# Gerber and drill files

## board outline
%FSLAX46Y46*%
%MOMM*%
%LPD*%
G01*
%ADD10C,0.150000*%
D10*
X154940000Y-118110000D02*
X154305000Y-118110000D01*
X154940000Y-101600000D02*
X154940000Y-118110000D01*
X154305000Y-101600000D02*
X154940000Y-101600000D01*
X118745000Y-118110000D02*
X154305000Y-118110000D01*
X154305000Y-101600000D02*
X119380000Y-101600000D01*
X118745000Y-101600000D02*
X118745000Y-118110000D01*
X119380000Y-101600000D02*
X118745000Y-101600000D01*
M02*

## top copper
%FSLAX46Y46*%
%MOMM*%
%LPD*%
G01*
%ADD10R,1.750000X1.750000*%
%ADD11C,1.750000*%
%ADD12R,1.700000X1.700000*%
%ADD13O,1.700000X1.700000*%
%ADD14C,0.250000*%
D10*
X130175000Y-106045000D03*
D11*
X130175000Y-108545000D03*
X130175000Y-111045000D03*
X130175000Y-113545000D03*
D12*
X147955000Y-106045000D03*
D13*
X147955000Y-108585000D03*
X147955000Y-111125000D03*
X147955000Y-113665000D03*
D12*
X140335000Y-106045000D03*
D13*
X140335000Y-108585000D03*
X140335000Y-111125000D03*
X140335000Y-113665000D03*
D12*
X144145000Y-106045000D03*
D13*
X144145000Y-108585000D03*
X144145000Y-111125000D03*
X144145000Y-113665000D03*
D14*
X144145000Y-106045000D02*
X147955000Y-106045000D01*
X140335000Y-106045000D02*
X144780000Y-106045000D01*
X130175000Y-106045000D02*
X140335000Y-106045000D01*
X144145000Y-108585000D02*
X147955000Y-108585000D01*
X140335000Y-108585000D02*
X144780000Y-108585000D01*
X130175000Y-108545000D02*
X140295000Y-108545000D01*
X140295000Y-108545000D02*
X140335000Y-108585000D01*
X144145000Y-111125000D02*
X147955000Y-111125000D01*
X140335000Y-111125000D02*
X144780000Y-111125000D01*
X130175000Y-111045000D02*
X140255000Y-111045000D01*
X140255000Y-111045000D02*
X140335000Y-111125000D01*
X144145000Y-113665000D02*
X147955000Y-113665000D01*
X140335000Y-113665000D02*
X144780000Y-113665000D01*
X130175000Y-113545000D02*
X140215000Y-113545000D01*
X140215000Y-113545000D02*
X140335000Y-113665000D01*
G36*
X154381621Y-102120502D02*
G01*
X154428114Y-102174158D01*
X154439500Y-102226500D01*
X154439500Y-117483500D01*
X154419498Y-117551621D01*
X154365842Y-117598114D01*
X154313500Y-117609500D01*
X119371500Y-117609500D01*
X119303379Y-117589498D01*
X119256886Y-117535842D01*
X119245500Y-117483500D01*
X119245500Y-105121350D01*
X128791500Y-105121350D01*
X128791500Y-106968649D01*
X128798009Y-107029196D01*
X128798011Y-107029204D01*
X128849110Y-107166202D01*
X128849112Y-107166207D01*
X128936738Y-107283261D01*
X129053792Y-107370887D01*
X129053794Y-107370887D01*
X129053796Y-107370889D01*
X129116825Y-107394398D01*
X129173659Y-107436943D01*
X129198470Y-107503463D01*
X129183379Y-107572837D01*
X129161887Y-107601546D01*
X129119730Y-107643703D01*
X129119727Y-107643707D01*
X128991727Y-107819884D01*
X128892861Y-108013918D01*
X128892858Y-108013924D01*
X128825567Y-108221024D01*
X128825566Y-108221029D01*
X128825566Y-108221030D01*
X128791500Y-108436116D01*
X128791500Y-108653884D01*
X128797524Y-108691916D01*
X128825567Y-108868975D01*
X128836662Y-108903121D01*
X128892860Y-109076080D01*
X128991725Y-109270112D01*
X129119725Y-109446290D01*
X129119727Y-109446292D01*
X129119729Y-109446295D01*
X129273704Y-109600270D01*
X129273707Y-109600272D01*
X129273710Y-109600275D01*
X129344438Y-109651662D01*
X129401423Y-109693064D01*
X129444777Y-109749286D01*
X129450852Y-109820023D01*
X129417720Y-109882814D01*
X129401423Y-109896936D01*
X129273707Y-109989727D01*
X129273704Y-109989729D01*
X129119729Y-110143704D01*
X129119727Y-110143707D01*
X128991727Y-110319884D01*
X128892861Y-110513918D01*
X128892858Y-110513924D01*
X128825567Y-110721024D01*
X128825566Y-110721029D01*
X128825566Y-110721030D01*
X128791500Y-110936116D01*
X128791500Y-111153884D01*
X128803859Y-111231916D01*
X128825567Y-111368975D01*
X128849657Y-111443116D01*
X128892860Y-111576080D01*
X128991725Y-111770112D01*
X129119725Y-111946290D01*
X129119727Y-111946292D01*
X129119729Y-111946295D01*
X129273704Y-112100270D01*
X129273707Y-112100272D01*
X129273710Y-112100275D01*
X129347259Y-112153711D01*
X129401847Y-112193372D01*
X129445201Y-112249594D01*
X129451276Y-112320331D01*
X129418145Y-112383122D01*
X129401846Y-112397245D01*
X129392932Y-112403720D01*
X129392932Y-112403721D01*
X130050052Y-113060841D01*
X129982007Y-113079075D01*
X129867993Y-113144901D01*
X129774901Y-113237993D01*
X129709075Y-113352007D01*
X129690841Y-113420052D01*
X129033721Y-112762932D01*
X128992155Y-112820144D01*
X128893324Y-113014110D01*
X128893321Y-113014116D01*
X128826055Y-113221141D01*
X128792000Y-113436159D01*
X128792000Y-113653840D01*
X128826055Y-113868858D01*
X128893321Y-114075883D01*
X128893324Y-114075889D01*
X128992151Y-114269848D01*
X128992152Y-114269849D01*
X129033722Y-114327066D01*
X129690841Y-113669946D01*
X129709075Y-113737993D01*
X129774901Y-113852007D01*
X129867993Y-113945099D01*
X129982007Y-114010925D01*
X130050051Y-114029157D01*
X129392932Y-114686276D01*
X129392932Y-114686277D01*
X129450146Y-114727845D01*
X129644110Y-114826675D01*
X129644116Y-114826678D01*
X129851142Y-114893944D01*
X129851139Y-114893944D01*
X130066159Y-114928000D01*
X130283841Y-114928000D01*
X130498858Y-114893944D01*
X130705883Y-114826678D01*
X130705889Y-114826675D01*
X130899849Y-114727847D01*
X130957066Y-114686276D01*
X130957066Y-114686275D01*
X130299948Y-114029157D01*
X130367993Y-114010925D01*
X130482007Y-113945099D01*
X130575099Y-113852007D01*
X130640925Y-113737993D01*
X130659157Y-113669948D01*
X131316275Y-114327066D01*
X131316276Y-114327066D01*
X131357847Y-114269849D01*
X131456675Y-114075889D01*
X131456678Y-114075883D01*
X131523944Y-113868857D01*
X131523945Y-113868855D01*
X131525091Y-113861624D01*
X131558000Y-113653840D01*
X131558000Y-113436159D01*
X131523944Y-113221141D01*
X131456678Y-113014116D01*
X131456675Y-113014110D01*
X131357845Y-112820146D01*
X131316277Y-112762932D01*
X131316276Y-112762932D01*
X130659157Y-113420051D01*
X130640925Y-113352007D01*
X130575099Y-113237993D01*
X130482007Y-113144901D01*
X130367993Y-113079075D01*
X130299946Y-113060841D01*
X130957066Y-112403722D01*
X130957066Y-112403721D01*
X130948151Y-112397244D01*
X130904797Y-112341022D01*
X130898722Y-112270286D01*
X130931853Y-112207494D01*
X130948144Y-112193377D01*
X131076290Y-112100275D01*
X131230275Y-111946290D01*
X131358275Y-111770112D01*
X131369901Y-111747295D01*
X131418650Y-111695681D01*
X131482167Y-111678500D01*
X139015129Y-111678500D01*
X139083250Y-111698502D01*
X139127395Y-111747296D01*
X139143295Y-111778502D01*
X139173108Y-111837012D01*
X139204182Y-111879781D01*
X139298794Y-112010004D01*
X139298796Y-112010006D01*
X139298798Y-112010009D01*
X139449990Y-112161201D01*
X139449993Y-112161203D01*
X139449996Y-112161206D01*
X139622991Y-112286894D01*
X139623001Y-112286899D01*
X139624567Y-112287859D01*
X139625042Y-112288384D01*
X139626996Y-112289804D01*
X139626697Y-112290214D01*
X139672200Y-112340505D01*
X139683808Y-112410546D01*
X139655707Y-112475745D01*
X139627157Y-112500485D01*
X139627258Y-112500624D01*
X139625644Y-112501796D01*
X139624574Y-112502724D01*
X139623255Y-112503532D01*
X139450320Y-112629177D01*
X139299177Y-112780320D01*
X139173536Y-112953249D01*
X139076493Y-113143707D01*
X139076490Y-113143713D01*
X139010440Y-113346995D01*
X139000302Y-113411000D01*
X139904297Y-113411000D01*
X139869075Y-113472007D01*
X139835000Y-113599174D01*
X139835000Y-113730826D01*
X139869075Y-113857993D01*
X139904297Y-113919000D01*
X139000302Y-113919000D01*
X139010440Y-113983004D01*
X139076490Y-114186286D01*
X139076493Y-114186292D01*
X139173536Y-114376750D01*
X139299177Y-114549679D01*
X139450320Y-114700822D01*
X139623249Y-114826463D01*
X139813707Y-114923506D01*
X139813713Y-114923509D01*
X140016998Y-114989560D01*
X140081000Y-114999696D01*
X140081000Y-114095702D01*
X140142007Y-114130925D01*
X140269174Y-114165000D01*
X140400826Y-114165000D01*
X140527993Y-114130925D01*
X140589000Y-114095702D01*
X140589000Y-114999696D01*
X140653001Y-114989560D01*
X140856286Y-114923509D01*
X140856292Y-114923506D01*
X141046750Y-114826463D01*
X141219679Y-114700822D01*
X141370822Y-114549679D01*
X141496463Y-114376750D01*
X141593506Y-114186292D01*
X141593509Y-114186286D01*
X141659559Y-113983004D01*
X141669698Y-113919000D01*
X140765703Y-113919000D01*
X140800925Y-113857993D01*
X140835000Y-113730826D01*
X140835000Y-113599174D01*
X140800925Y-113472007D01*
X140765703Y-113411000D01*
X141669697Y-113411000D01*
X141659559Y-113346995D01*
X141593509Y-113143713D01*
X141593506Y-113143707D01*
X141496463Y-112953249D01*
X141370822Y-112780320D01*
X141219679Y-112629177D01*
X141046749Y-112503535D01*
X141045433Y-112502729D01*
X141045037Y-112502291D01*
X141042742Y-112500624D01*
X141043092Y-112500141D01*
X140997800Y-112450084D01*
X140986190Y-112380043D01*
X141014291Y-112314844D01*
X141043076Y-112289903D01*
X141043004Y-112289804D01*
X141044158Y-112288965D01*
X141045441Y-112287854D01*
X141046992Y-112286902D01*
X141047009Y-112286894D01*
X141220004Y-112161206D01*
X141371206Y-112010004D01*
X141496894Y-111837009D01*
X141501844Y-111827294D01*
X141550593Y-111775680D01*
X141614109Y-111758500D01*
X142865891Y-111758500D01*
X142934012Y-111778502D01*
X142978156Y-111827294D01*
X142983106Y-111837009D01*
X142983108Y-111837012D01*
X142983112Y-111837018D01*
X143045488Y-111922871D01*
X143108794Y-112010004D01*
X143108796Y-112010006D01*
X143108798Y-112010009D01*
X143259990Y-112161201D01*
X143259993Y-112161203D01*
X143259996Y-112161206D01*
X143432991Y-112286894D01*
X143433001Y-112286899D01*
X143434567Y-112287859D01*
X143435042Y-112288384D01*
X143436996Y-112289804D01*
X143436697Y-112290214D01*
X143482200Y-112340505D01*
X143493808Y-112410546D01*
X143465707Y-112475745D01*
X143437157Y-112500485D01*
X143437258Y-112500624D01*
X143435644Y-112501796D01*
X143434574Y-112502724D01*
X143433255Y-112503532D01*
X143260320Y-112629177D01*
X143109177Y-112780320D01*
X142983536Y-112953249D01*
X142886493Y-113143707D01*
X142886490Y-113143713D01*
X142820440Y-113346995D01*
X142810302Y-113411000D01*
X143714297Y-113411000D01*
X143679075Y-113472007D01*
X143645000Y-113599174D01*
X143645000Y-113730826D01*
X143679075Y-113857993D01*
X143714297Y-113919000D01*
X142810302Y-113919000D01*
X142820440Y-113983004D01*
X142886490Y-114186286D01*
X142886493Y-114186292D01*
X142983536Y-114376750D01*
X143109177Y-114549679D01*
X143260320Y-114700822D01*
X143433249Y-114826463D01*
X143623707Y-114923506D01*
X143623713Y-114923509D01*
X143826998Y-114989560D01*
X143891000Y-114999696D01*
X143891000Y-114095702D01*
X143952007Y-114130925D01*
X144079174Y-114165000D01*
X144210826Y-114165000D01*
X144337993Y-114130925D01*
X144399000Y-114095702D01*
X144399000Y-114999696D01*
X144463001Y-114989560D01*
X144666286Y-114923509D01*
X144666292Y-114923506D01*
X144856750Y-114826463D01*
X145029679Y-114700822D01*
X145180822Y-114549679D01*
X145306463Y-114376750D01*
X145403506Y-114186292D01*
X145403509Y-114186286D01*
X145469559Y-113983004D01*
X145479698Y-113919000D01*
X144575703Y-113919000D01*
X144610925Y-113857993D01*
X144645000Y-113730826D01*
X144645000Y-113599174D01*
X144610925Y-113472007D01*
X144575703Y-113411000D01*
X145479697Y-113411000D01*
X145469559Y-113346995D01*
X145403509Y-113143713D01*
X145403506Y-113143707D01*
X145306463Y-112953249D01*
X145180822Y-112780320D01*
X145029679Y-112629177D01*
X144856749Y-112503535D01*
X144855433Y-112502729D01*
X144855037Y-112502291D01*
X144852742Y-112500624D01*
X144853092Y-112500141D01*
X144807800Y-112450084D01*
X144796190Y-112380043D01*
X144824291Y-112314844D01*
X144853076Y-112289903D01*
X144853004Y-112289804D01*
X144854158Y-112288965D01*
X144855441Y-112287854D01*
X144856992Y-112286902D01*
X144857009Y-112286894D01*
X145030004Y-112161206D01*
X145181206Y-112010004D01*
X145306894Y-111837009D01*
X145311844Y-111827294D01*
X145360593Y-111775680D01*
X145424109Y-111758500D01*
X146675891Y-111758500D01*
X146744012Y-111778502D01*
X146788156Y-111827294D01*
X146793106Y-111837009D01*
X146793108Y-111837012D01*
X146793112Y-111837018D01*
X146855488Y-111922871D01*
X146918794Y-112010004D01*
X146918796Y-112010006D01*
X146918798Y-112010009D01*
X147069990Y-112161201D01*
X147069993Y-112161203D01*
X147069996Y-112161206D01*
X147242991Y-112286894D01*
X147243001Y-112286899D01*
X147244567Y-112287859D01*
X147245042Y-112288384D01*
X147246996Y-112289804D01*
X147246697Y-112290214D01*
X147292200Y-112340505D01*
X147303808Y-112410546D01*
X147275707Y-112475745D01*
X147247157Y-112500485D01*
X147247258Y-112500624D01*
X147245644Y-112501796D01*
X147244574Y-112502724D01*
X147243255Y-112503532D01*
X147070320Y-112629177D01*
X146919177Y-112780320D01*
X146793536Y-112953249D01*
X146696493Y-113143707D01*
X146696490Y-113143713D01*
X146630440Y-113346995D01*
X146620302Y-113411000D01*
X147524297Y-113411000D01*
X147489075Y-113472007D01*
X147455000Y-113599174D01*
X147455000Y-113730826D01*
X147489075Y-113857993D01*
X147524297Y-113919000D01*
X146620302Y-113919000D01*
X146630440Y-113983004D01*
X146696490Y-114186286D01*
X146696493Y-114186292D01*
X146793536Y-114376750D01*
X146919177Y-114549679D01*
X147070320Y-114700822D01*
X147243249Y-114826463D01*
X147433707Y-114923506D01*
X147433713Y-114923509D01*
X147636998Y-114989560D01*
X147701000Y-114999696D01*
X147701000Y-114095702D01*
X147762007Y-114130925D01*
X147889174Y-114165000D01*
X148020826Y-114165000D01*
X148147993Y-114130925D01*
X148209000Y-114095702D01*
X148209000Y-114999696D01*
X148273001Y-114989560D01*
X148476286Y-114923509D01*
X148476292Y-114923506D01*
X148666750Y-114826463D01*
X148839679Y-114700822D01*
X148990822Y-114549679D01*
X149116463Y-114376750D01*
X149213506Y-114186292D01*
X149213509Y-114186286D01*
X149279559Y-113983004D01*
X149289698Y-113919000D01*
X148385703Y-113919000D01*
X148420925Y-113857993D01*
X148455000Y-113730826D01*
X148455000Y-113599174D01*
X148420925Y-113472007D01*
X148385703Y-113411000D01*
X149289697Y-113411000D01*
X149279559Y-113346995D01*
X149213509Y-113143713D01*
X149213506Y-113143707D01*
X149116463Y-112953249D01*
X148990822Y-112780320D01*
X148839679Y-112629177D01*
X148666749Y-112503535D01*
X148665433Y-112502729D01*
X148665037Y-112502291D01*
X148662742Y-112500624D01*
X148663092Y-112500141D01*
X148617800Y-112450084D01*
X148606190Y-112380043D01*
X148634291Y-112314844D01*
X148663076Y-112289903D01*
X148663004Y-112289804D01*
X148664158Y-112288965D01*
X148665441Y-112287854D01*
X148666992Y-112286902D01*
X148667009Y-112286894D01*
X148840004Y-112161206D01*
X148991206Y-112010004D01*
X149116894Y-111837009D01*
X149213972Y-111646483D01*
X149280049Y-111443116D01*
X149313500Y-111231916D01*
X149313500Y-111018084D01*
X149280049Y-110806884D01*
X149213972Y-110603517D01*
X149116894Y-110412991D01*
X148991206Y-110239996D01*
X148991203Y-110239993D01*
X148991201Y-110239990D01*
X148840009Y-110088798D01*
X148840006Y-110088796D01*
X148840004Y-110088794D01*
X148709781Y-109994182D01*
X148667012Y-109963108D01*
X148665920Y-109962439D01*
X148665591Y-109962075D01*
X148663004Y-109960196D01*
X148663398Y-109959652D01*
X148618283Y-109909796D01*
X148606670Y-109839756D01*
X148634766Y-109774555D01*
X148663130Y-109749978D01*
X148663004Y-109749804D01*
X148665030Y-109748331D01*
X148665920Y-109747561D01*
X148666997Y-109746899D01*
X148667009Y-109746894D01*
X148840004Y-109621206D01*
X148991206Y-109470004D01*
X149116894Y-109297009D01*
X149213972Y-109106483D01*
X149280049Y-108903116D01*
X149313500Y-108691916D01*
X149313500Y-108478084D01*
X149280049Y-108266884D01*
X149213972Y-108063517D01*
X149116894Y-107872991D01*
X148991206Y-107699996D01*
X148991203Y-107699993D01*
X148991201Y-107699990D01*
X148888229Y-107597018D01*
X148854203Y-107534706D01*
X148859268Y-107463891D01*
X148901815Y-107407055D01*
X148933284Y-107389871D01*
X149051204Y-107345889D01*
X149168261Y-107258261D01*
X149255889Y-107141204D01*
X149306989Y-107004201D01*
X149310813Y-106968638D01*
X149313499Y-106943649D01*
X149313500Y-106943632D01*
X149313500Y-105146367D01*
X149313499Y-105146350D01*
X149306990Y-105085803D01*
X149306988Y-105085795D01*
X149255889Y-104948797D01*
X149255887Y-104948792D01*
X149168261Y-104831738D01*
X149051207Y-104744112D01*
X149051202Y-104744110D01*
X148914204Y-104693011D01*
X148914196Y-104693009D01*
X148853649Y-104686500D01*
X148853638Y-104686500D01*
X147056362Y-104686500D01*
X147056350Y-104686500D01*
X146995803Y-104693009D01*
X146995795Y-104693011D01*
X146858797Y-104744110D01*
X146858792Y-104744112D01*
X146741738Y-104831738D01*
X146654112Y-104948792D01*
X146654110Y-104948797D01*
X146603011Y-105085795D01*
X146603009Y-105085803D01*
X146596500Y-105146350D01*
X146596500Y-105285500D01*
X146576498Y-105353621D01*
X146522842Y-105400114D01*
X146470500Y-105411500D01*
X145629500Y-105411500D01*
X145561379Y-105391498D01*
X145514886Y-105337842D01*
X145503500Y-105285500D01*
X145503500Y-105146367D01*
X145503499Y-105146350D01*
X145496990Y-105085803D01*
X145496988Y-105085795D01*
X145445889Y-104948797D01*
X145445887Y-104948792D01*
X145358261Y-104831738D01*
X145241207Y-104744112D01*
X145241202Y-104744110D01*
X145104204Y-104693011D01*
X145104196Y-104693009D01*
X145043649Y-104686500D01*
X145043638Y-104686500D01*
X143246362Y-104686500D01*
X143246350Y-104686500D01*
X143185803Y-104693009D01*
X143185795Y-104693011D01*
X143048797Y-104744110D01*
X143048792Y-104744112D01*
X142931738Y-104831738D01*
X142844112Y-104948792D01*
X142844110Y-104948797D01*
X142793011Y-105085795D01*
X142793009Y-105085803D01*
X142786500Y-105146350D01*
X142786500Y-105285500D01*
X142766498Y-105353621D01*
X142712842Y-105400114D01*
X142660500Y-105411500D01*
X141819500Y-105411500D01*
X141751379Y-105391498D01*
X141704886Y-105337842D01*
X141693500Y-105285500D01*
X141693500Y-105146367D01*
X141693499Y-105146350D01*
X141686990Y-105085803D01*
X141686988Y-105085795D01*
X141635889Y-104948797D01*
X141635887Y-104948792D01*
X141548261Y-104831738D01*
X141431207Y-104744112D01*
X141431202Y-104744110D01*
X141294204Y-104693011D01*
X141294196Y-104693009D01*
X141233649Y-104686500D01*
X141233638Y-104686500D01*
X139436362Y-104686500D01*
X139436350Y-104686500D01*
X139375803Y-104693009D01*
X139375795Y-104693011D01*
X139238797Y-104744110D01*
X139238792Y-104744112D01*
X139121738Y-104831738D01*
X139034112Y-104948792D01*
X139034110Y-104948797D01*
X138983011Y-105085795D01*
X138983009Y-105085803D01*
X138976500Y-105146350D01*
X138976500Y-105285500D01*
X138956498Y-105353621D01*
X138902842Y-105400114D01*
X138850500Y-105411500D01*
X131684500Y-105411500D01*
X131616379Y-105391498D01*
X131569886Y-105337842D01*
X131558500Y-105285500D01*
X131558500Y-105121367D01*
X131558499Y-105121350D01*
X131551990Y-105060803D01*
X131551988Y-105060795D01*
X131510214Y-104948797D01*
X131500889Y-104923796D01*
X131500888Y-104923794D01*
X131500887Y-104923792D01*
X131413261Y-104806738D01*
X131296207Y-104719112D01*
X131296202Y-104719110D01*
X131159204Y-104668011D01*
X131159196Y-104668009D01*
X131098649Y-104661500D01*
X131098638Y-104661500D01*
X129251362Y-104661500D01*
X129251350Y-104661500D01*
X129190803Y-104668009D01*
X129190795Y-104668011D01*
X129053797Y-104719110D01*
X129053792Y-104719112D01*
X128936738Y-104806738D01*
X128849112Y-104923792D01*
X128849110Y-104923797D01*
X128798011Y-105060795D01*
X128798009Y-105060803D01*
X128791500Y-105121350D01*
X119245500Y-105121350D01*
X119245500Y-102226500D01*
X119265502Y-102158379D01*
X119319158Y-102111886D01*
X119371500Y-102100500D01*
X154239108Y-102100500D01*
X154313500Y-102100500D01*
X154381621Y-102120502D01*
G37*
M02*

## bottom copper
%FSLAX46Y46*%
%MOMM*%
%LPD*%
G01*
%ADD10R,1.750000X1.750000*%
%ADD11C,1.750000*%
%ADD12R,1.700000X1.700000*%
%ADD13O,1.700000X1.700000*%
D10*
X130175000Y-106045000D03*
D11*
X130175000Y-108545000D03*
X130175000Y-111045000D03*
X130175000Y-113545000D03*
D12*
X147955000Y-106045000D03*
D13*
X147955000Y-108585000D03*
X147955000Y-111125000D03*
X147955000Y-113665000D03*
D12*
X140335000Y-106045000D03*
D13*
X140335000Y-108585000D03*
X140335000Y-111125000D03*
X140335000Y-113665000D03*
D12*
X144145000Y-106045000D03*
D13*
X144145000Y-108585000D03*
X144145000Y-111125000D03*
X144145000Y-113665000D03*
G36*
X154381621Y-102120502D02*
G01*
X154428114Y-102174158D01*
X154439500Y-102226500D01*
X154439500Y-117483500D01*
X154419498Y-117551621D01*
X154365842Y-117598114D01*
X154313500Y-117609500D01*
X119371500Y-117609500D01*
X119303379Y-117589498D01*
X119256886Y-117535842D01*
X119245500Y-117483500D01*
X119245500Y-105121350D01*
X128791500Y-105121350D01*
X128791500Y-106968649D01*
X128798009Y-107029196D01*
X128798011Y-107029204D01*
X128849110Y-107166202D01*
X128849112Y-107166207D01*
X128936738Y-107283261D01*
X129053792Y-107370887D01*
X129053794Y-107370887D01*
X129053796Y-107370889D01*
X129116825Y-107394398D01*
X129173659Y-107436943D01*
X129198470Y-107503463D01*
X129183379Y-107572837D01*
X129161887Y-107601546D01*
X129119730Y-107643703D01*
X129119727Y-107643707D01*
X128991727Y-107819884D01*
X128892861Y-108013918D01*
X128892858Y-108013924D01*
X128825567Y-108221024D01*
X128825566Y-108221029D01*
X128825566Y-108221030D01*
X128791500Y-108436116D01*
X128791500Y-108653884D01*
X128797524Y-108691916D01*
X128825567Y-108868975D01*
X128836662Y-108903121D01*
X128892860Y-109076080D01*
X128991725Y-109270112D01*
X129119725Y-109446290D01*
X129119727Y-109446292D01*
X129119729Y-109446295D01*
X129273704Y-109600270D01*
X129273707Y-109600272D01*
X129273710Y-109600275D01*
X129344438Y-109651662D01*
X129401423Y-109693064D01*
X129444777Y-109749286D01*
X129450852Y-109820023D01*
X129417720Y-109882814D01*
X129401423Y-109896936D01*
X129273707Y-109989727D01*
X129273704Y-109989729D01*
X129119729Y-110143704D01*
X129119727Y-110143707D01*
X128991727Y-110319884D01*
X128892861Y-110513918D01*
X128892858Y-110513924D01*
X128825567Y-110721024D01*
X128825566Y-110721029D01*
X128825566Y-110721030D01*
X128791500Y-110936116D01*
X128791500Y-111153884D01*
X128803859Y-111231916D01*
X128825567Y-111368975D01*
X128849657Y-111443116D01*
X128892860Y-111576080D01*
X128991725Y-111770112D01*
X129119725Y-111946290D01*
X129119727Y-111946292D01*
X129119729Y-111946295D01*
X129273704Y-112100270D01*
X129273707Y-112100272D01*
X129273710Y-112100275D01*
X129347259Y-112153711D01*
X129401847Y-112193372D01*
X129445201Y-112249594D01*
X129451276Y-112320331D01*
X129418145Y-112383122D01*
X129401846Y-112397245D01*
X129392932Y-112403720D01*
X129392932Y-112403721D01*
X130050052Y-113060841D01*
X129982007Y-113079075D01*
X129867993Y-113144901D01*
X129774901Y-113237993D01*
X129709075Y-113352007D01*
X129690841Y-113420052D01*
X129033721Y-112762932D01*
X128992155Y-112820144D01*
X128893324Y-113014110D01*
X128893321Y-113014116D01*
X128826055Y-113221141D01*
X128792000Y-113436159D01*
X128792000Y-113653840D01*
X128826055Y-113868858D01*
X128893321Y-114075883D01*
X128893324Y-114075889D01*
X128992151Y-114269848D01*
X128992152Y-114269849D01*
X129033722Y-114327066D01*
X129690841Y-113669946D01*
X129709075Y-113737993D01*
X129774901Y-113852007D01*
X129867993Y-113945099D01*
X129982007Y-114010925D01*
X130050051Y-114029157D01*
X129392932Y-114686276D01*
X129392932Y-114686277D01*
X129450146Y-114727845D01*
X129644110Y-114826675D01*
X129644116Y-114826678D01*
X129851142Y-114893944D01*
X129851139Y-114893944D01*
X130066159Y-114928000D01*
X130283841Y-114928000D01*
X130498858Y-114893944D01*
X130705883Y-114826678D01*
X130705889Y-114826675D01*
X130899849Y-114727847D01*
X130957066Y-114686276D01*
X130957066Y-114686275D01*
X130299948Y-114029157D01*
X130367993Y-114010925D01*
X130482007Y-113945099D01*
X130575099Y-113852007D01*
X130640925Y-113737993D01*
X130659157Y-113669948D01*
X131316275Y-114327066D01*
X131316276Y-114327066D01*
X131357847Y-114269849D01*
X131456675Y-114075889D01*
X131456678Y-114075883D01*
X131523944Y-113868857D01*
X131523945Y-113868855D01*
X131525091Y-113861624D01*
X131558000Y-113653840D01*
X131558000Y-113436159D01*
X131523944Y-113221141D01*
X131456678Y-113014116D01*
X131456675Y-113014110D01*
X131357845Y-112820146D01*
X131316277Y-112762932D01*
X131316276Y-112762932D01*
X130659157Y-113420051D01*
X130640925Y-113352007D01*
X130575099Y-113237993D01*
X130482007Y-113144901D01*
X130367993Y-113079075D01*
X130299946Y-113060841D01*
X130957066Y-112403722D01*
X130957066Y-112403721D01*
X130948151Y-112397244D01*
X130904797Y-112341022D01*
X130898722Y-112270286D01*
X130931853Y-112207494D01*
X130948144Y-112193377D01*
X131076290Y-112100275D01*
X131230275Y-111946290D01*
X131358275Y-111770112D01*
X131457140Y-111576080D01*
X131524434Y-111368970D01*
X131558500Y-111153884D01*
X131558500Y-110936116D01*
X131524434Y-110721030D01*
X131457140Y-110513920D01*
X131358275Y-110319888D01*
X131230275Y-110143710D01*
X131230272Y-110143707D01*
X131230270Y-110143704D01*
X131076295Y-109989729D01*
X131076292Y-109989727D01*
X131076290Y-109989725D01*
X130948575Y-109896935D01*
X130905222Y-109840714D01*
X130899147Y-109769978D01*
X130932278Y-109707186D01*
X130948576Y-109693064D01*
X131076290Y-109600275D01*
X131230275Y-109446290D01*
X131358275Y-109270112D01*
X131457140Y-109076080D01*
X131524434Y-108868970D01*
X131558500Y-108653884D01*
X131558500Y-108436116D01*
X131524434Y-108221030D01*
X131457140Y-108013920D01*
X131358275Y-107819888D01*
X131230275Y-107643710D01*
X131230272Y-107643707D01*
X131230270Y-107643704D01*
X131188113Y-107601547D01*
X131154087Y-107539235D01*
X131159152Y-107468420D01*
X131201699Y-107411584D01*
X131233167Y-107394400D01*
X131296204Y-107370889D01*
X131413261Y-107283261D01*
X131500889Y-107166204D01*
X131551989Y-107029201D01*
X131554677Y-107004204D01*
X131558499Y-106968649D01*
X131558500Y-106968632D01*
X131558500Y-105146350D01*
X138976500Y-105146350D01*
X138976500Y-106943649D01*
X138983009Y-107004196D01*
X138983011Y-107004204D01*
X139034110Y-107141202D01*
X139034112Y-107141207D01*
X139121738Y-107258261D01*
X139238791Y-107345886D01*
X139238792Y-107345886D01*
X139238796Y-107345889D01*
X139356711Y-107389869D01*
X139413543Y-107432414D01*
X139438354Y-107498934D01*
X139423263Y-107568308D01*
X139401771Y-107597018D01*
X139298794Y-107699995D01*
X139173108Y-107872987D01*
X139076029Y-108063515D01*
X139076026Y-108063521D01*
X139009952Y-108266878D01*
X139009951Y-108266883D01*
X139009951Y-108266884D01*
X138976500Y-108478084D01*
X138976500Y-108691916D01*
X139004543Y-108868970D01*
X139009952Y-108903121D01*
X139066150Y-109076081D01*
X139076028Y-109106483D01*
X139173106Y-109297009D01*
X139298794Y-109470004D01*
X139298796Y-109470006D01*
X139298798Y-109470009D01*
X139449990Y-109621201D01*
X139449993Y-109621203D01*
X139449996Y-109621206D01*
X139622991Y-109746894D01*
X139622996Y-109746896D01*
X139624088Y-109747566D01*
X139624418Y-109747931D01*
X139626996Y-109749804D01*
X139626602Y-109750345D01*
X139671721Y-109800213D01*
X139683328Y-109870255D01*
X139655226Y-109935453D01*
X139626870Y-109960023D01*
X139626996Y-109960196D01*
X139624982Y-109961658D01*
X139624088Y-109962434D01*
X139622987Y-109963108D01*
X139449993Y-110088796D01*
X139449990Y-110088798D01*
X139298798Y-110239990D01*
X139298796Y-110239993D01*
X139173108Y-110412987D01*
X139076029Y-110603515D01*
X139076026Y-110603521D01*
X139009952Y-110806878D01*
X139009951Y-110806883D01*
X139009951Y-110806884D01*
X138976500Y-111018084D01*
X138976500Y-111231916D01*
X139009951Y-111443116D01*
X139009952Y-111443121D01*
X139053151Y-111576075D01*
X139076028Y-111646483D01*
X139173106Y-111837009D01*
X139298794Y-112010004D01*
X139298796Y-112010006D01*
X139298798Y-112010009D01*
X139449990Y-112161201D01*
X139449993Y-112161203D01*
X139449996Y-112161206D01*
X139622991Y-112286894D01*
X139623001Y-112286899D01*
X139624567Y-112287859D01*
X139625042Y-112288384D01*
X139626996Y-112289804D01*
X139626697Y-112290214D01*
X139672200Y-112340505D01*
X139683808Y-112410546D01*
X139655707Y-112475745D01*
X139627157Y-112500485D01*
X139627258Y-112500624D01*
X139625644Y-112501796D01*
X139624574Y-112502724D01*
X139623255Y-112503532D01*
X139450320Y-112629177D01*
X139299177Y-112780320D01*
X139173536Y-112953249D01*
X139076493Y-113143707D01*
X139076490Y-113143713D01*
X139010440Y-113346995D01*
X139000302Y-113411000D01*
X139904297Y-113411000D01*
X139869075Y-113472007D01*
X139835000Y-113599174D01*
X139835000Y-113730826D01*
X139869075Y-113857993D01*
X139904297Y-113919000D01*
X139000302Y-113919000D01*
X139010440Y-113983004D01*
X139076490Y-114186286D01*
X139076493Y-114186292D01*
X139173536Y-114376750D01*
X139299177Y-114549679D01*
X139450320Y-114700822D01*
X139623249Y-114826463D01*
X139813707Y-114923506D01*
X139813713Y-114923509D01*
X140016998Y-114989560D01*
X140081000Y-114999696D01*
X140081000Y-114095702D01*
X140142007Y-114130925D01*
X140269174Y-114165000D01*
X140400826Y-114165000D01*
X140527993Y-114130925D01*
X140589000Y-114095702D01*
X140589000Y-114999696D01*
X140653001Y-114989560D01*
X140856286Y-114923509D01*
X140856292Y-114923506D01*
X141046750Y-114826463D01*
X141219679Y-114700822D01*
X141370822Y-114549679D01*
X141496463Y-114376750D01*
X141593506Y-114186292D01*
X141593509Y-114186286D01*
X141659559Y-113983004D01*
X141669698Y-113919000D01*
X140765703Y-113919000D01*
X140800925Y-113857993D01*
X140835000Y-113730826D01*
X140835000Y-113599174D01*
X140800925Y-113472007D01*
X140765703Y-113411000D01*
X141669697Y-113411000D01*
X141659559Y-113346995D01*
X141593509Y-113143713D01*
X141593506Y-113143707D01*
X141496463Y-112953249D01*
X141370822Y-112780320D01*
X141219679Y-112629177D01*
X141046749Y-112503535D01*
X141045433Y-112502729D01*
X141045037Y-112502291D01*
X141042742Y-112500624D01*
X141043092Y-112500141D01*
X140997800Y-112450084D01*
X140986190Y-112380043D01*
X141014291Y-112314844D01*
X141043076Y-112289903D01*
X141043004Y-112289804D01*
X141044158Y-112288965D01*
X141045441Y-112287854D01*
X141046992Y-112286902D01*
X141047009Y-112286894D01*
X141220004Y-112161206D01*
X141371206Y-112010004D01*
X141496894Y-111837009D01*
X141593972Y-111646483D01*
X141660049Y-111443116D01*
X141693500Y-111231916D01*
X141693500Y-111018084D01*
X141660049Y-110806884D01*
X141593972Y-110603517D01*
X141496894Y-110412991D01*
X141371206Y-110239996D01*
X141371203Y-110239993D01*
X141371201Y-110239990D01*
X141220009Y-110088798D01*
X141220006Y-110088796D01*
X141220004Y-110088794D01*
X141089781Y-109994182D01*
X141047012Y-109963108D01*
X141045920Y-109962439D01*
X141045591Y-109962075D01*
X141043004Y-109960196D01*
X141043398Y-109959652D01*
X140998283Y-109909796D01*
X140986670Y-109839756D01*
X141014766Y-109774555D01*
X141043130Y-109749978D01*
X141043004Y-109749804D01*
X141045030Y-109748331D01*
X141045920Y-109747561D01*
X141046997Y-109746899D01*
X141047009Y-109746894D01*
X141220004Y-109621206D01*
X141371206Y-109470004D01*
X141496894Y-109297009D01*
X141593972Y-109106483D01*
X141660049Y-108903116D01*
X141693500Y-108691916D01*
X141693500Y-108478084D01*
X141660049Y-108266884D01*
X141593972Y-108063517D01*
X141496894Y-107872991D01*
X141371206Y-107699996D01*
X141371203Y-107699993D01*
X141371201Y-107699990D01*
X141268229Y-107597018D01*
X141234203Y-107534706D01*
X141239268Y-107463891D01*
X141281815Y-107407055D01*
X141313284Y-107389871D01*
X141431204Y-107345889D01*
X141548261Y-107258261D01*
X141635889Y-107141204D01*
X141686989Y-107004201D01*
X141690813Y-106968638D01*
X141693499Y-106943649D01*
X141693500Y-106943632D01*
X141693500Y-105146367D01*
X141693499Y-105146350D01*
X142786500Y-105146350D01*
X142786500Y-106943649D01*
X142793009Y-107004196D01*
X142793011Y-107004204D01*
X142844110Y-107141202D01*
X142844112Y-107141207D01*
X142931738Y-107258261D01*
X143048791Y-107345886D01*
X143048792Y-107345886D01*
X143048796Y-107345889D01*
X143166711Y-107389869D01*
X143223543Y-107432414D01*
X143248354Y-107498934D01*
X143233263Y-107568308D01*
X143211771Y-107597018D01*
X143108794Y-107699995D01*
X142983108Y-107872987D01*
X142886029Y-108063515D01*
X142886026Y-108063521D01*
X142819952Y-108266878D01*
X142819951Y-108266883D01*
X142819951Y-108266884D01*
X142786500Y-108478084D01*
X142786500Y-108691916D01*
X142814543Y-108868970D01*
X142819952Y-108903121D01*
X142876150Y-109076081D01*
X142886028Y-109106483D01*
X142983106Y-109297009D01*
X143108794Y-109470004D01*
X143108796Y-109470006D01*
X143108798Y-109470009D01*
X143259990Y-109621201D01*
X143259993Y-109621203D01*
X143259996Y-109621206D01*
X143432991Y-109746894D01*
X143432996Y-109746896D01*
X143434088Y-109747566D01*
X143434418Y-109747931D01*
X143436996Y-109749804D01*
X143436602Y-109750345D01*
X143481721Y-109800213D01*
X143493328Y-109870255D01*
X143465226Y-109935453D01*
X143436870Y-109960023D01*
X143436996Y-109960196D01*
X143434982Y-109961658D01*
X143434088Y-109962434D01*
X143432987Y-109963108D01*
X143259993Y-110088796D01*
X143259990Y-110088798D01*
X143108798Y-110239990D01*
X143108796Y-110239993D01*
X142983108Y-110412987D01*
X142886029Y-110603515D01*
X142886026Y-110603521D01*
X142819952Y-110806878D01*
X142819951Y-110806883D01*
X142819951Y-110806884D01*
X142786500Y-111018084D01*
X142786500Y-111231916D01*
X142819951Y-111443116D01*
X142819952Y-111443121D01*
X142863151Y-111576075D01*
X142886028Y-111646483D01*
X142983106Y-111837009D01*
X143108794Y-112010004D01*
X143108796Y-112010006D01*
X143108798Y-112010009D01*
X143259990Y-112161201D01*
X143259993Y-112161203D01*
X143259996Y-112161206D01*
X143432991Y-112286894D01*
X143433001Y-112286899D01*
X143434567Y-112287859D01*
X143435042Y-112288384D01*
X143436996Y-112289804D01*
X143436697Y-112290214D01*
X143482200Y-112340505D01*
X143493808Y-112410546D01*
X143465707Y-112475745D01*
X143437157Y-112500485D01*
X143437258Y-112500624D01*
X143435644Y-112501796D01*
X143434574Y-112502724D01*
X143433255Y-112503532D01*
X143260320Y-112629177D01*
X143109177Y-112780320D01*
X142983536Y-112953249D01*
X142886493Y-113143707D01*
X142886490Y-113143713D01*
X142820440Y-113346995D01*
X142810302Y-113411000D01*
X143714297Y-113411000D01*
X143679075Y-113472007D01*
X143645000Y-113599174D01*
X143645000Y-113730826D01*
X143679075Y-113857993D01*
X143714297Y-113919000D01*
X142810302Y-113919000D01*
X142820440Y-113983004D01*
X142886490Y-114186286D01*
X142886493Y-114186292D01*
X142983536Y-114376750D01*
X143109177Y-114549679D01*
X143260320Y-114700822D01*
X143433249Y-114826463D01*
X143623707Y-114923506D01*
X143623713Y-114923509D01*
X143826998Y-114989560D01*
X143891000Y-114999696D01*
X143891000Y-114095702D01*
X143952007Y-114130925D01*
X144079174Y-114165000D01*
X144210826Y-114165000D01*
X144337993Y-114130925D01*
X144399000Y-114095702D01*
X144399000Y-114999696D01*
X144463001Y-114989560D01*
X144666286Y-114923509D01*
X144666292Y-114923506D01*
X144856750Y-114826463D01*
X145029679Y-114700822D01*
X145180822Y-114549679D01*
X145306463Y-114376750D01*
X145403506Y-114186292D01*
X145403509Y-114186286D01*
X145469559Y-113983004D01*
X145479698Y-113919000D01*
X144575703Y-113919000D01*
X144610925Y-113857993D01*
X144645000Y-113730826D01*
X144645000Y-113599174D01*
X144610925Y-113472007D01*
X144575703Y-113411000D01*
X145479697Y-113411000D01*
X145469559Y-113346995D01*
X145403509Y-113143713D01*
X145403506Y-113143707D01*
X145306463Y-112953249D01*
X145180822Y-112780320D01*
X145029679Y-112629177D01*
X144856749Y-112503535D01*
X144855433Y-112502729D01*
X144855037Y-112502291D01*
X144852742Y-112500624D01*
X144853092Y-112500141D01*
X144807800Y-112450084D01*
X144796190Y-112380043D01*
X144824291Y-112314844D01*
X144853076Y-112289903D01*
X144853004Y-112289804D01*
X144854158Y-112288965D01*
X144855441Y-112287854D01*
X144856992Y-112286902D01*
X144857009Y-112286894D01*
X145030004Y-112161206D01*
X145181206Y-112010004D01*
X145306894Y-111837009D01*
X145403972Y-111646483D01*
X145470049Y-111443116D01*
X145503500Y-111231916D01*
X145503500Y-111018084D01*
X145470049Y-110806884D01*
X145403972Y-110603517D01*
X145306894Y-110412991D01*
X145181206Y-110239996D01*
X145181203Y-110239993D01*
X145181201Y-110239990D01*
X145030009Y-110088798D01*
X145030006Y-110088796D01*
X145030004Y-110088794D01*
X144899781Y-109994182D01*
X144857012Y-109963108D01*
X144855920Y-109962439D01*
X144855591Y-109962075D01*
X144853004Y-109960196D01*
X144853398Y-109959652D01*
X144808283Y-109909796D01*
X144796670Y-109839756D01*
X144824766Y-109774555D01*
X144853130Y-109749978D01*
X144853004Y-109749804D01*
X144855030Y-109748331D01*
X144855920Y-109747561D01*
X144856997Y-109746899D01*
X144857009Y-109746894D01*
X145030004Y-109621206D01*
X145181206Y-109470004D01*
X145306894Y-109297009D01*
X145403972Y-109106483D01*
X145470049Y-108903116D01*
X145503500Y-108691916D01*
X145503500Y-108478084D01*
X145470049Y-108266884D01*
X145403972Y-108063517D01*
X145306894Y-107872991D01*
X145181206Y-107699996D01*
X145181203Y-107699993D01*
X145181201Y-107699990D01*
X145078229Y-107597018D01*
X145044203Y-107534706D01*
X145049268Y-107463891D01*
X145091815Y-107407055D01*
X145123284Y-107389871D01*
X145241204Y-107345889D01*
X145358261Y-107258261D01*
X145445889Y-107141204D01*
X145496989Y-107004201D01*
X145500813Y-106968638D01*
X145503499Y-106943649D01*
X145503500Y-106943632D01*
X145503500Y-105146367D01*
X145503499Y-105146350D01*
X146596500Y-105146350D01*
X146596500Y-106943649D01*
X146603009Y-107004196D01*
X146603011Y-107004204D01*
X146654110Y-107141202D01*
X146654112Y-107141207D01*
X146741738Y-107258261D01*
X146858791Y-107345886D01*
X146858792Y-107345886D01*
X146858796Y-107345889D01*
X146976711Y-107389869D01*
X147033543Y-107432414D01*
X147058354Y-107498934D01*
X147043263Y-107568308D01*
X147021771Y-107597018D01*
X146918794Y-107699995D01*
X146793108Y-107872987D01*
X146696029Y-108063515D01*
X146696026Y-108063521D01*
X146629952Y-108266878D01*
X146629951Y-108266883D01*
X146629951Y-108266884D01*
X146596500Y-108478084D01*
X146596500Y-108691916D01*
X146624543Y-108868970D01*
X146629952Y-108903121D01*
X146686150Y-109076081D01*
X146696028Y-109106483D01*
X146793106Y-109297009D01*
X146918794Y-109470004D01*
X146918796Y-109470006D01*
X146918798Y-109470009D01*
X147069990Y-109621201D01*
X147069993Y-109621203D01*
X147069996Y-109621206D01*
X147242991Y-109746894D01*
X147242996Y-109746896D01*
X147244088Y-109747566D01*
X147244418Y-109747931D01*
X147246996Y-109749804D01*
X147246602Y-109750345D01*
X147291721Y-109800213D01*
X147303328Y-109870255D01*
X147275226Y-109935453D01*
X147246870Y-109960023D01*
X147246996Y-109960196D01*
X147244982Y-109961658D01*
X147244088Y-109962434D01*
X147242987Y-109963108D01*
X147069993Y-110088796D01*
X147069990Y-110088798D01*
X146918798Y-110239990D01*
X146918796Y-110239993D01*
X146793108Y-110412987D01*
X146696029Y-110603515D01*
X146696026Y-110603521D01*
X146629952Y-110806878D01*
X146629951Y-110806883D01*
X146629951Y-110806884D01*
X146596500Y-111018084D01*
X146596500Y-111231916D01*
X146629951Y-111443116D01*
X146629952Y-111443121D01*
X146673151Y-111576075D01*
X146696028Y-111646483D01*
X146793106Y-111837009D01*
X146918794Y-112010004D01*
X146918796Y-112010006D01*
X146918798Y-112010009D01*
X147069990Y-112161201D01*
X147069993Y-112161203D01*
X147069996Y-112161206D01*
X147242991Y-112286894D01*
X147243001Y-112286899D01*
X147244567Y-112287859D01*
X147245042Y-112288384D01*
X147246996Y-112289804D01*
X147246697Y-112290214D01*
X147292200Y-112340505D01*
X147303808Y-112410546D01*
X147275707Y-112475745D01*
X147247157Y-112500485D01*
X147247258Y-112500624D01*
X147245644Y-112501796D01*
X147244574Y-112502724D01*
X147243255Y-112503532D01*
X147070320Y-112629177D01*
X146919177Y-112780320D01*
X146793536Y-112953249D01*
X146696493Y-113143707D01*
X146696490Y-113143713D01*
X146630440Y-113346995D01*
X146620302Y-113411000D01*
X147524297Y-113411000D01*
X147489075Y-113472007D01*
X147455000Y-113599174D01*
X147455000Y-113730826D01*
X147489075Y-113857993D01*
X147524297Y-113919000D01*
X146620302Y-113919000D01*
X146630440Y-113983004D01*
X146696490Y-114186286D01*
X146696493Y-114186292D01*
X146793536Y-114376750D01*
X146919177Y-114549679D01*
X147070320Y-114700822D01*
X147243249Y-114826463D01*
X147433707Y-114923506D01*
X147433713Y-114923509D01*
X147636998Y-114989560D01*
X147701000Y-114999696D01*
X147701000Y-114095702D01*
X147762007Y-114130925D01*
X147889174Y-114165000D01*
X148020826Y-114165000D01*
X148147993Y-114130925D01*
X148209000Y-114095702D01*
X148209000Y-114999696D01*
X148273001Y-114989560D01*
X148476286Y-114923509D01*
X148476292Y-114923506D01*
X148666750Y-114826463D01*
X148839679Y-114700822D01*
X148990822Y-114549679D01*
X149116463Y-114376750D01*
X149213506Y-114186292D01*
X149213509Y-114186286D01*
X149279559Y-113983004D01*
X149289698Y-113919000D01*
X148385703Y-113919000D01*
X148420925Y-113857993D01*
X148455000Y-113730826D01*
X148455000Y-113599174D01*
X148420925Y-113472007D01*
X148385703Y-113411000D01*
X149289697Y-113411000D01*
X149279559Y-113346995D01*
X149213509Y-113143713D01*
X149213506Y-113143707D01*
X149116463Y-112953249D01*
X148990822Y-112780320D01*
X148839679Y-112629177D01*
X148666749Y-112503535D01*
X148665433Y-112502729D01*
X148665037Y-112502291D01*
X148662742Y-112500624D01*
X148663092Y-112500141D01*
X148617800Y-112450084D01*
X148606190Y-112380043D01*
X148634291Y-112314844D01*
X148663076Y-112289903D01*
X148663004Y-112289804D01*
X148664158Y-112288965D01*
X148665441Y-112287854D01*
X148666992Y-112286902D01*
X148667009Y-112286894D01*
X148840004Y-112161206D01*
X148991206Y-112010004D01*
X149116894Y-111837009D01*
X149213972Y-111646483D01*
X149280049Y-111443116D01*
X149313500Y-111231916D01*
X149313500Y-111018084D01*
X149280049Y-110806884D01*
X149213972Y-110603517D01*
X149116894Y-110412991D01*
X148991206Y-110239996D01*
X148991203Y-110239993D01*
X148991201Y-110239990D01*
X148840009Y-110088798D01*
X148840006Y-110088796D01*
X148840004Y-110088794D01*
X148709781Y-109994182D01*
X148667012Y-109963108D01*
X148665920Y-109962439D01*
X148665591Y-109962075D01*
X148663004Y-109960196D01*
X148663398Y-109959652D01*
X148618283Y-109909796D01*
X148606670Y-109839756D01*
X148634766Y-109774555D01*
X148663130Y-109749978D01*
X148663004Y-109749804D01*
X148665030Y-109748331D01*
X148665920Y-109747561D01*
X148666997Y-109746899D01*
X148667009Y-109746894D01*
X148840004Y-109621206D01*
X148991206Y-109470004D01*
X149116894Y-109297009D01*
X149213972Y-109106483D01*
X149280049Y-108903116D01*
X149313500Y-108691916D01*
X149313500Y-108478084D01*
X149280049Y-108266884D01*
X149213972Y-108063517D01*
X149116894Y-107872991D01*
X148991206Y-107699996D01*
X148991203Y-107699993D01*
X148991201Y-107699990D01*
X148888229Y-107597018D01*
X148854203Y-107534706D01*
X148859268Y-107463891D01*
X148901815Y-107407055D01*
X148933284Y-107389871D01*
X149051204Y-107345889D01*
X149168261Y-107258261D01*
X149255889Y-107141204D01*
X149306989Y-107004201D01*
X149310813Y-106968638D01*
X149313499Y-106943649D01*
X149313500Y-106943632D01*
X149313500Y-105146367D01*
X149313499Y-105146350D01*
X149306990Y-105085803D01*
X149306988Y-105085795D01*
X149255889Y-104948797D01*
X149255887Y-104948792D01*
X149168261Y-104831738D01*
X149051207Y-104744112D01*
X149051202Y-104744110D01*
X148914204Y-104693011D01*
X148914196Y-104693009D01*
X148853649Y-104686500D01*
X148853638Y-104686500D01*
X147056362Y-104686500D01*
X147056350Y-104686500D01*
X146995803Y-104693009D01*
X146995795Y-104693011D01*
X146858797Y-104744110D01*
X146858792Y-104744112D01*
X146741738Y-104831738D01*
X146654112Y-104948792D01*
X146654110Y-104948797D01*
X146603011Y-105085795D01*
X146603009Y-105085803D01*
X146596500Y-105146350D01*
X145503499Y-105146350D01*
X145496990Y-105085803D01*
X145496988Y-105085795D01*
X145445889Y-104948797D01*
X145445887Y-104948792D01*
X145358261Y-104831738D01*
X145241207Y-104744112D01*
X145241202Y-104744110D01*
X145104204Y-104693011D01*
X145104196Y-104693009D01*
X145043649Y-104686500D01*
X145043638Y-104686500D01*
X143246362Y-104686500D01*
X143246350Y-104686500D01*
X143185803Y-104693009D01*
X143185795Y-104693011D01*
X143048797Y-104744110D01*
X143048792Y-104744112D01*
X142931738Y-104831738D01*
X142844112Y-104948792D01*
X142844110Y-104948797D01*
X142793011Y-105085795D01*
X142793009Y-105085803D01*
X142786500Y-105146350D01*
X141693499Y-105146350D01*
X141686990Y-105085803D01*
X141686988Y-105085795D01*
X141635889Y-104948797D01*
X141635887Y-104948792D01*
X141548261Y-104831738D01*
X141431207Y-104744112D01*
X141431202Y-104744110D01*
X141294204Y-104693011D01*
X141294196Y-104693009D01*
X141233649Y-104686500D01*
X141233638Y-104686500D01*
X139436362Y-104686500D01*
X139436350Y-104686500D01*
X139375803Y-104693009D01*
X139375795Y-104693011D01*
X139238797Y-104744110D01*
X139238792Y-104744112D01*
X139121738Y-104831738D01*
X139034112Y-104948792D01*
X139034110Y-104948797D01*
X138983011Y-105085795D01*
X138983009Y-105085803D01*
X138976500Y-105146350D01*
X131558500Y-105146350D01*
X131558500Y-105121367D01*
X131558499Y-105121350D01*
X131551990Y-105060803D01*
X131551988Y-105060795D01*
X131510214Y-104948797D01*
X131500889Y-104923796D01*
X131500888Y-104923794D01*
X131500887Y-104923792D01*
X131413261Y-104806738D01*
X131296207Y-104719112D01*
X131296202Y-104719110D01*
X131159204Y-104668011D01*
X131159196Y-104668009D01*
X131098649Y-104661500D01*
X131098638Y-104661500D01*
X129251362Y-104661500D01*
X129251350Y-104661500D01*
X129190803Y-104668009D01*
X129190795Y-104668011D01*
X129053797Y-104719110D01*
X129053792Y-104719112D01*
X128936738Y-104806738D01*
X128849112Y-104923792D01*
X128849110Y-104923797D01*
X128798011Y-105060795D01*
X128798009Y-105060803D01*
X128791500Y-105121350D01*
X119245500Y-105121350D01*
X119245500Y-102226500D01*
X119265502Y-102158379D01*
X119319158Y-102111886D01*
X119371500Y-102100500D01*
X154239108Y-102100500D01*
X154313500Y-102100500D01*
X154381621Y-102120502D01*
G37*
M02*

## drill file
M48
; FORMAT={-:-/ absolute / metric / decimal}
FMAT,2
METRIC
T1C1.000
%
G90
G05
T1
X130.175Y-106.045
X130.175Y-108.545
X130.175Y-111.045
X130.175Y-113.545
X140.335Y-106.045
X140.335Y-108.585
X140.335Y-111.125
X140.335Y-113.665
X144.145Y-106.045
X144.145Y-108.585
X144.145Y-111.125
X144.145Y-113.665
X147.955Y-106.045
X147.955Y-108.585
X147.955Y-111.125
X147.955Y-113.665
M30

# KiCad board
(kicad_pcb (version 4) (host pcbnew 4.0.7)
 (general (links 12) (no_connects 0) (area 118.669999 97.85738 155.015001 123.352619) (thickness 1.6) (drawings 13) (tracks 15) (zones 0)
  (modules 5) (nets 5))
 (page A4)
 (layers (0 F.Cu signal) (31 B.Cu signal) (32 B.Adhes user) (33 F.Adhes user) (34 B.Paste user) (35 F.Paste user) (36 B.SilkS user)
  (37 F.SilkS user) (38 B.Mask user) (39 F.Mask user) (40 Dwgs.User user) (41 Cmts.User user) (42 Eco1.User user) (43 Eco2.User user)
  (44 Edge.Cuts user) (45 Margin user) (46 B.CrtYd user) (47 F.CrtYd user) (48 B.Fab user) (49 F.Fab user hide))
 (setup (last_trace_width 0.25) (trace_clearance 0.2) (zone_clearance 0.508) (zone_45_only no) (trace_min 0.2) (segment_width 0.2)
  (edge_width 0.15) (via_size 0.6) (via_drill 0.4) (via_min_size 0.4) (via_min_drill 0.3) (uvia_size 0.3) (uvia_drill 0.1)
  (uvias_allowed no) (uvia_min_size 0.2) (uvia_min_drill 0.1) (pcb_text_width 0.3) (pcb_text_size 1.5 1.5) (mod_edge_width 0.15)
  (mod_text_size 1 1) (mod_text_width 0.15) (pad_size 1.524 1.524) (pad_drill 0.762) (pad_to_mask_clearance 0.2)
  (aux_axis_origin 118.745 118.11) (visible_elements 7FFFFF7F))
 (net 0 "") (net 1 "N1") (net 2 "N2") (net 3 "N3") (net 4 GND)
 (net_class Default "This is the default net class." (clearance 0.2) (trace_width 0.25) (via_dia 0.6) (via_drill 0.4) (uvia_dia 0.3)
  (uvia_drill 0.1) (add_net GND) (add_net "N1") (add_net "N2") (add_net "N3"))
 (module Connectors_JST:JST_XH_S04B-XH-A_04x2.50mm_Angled (layer F.Cu) (at 130.175 106.045 270)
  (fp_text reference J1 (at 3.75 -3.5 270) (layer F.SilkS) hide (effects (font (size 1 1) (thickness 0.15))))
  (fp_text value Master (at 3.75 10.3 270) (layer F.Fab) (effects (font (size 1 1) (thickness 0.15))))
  (pad 1 thru_hole rect (at 0 0 270) (size 1.75 1.75) (drill 1) (layers *.Cu *.Mask F.SilkS) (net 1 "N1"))
  (pad 2 thru_hole circle (at 2.5 0 270) (size 1.75 1.75) (drill 1) (layers *.Cu *.Mask F.SilkS) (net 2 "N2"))
  (pad 3 thru_hole circle (at 5 0 270) (size 1.75 1.75) (drill 1) (layers *.Cu *.Mask F.SilkS) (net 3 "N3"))
  (pad 4 thru_hole circle (at 7.5 0 270) (size 1.75 1.75) (drill 1) (layers *.Cu *.Mask F.SilkS) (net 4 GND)))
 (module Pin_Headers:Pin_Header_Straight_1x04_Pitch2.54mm (layer F.Cu) (at 147.955 106.045)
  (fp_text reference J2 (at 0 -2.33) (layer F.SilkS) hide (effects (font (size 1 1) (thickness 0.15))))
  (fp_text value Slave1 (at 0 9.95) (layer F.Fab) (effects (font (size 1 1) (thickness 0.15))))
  (pad 1 thru_hole rect (at 0 0) (size 1.7 1.7) (drill 1) (layers *.Cu *.Mask) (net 1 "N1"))
  (pad 2 thru_hole oval (at 0 2.54) (size 1.7 1.7) (drill 1) (layers *.Cu *.Mask) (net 2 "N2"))
  (pad 3 thru_hole oval (at 0 5.08) (size 1.7 1.7) (drill 1) (layers *.Cu *.Mask) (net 3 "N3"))
  (pad 4 thru_hole oval (at 0 7.62) (size 1.7 1.7) (drill 1) (layers *.Cu *.Mask) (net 4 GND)))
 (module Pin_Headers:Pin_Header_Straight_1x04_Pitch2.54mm (layer F.Cu) (at 140.335 106.045)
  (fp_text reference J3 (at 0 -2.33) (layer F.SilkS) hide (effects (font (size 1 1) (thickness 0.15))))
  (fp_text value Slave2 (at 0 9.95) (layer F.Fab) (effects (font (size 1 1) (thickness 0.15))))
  (pad 1 thru_hole rect (at 0 0) (size 1.7 1.7) (drill 1) (layers *.Cu *.Mask) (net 1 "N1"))
  (pad 2 thru_hole oval (at 0 2.54) (size 1.7 1.7) (drill 1) (layers *.Cu *.Mask) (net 2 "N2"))
  (pad 3 thru_hole oval (at 0 5.08) (size 1.7 1.7) (drill 1) (layers *.Cu *.Mask) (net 3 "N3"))
  (pad 4 thru_hole oval (at 0 7.62) (size 1.7 1.7) (drill 1) (layers *.Cu *.Mask) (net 4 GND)))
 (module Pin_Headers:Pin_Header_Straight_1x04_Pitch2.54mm (layer F.Cu) (at 144.145 106.045)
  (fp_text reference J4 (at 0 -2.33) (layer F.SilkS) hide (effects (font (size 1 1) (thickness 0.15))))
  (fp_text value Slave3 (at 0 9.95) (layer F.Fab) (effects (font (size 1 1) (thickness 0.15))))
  (pad 1 thru_hole rect (at 0 0) (size 1.7 1.7) (drill 1) (layers *.Cu *.Mask) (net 1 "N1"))
  (pad 2 thru_hole oval (at 0 2.54) (size 1.7 1.7) (drill 1) (layers *.Cu *.Mask) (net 2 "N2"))
  (pad 3 thru_hole oval (at 0 5.08) (size 1.7 1.7) (drill 1) (layers *.Cu *.Mask) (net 3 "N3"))
  (pad 4 thru_hole oval (at 0 7.62) (size 1.7 1.7) (drill 1) (layers *.Cu *.Mask) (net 4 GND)))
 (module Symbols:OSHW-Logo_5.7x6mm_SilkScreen (layer B.Cu) (at 135.255 109.855 270)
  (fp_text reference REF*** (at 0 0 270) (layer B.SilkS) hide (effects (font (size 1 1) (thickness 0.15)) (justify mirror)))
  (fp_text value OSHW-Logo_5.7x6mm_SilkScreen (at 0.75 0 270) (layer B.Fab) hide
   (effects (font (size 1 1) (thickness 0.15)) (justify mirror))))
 (gr_line (start 154.94 118.11) (end 154.305 118.11) (layer Edge.Cuts) (width 0.15))
 (gr_line (start 154.94 101.6) (end 154.94 118.11) (layer Edge.Cuts) (width 0.15))
 (gr_line (start 154.305 101.6) (end 154.94 101.6) (layer Edge.Cuts) (width 0.15))
 (gr_line (start 118.745 118.11) (end 154.305 118.11) (layer Edge.Cuts) (width 0.15))
 (gr_line (start 154.305 101.6) (end 119.38 101.6) (layer Edge.Cuts) (width 0.15))
 (gr_line (start 118.745 101.6) (end 118.745 118.11) (layer Edge.Cuts) (width 0.15))
 (gr_line (start 119.38 101.6) (end 118.745 101.6) (layer Edge.Cuts) (width 0.15))
 (segment (start 144.145 106.045) (end 147.955 106.045) (width 0.25) (layer F.Cu) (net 1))
 (segment (start 140.335 106.045) (end 144.78 106.045) (width 0.25) (layer F.Cu) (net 1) (status 30))
 (segment (start 130.175 106.045) (end 140.335 106.045) (width 0.25) (layer F.Cu) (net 1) (status 30))
 (segment (start 144.145 108.585) (end 147.955 108.585) (width 0.25) (layer F.Cu) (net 2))
 (segment (start 140.335 108.585) (end 144.78 108.585) (width 0.25) (layer F.Cu) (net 2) (status 30))
 (segment (start 130.175 108.545) (end 140.295 108.545) (width 0.25) (layer F.Cu) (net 2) (status 30))
 (segment (start 140.295 108.545) (end 140.335 108.585) (width 0.25) (layer F.Cu) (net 2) (status 30))
 (segment (start 144.145 111.125) (end 147.955 111.125) (width 0.25) (layer F.Cu) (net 3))
 (segment (start 140.335 111.125) (end 144.78 111.125) (width 0.25) (layer F.Cu) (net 3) (status 30))
 (segment (start 130.175 111.045) (end 140.255 111.045) (width 0.25) (layer F.Cu) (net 3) (status 30))
 (segment (start 140.255 111.045) (end 140.335 111.125) (width 0.25) (layer F.Cu) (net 3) (status 30))
 (segment (start 144.145 113.665) (end 147.955 113.665) (width 0.25) (layer F.Cu) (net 4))
 (segment (start 140.335 113.665) (end 144.78 113.665) (width 0.25) (layer F.Cu) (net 4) (status 30))
 (segment (start 130.175 113.545) (end 140.215 113.545) (width 0.25) (layer F.Cu) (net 4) (status 30))
 (segment (start 140.215 113.545) (end 140.335 113.665) (width 0.25) (layer F.Cu) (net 4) (status 30))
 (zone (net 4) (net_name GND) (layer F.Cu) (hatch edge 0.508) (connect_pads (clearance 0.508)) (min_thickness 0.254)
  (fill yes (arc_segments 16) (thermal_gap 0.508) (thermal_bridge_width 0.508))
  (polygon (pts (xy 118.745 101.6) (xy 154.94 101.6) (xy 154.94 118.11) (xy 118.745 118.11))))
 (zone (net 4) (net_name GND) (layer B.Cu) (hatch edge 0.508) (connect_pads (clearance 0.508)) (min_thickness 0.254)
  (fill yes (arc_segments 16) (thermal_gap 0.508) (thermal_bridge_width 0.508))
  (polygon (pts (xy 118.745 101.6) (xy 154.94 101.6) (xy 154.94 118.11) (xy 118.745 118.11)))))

